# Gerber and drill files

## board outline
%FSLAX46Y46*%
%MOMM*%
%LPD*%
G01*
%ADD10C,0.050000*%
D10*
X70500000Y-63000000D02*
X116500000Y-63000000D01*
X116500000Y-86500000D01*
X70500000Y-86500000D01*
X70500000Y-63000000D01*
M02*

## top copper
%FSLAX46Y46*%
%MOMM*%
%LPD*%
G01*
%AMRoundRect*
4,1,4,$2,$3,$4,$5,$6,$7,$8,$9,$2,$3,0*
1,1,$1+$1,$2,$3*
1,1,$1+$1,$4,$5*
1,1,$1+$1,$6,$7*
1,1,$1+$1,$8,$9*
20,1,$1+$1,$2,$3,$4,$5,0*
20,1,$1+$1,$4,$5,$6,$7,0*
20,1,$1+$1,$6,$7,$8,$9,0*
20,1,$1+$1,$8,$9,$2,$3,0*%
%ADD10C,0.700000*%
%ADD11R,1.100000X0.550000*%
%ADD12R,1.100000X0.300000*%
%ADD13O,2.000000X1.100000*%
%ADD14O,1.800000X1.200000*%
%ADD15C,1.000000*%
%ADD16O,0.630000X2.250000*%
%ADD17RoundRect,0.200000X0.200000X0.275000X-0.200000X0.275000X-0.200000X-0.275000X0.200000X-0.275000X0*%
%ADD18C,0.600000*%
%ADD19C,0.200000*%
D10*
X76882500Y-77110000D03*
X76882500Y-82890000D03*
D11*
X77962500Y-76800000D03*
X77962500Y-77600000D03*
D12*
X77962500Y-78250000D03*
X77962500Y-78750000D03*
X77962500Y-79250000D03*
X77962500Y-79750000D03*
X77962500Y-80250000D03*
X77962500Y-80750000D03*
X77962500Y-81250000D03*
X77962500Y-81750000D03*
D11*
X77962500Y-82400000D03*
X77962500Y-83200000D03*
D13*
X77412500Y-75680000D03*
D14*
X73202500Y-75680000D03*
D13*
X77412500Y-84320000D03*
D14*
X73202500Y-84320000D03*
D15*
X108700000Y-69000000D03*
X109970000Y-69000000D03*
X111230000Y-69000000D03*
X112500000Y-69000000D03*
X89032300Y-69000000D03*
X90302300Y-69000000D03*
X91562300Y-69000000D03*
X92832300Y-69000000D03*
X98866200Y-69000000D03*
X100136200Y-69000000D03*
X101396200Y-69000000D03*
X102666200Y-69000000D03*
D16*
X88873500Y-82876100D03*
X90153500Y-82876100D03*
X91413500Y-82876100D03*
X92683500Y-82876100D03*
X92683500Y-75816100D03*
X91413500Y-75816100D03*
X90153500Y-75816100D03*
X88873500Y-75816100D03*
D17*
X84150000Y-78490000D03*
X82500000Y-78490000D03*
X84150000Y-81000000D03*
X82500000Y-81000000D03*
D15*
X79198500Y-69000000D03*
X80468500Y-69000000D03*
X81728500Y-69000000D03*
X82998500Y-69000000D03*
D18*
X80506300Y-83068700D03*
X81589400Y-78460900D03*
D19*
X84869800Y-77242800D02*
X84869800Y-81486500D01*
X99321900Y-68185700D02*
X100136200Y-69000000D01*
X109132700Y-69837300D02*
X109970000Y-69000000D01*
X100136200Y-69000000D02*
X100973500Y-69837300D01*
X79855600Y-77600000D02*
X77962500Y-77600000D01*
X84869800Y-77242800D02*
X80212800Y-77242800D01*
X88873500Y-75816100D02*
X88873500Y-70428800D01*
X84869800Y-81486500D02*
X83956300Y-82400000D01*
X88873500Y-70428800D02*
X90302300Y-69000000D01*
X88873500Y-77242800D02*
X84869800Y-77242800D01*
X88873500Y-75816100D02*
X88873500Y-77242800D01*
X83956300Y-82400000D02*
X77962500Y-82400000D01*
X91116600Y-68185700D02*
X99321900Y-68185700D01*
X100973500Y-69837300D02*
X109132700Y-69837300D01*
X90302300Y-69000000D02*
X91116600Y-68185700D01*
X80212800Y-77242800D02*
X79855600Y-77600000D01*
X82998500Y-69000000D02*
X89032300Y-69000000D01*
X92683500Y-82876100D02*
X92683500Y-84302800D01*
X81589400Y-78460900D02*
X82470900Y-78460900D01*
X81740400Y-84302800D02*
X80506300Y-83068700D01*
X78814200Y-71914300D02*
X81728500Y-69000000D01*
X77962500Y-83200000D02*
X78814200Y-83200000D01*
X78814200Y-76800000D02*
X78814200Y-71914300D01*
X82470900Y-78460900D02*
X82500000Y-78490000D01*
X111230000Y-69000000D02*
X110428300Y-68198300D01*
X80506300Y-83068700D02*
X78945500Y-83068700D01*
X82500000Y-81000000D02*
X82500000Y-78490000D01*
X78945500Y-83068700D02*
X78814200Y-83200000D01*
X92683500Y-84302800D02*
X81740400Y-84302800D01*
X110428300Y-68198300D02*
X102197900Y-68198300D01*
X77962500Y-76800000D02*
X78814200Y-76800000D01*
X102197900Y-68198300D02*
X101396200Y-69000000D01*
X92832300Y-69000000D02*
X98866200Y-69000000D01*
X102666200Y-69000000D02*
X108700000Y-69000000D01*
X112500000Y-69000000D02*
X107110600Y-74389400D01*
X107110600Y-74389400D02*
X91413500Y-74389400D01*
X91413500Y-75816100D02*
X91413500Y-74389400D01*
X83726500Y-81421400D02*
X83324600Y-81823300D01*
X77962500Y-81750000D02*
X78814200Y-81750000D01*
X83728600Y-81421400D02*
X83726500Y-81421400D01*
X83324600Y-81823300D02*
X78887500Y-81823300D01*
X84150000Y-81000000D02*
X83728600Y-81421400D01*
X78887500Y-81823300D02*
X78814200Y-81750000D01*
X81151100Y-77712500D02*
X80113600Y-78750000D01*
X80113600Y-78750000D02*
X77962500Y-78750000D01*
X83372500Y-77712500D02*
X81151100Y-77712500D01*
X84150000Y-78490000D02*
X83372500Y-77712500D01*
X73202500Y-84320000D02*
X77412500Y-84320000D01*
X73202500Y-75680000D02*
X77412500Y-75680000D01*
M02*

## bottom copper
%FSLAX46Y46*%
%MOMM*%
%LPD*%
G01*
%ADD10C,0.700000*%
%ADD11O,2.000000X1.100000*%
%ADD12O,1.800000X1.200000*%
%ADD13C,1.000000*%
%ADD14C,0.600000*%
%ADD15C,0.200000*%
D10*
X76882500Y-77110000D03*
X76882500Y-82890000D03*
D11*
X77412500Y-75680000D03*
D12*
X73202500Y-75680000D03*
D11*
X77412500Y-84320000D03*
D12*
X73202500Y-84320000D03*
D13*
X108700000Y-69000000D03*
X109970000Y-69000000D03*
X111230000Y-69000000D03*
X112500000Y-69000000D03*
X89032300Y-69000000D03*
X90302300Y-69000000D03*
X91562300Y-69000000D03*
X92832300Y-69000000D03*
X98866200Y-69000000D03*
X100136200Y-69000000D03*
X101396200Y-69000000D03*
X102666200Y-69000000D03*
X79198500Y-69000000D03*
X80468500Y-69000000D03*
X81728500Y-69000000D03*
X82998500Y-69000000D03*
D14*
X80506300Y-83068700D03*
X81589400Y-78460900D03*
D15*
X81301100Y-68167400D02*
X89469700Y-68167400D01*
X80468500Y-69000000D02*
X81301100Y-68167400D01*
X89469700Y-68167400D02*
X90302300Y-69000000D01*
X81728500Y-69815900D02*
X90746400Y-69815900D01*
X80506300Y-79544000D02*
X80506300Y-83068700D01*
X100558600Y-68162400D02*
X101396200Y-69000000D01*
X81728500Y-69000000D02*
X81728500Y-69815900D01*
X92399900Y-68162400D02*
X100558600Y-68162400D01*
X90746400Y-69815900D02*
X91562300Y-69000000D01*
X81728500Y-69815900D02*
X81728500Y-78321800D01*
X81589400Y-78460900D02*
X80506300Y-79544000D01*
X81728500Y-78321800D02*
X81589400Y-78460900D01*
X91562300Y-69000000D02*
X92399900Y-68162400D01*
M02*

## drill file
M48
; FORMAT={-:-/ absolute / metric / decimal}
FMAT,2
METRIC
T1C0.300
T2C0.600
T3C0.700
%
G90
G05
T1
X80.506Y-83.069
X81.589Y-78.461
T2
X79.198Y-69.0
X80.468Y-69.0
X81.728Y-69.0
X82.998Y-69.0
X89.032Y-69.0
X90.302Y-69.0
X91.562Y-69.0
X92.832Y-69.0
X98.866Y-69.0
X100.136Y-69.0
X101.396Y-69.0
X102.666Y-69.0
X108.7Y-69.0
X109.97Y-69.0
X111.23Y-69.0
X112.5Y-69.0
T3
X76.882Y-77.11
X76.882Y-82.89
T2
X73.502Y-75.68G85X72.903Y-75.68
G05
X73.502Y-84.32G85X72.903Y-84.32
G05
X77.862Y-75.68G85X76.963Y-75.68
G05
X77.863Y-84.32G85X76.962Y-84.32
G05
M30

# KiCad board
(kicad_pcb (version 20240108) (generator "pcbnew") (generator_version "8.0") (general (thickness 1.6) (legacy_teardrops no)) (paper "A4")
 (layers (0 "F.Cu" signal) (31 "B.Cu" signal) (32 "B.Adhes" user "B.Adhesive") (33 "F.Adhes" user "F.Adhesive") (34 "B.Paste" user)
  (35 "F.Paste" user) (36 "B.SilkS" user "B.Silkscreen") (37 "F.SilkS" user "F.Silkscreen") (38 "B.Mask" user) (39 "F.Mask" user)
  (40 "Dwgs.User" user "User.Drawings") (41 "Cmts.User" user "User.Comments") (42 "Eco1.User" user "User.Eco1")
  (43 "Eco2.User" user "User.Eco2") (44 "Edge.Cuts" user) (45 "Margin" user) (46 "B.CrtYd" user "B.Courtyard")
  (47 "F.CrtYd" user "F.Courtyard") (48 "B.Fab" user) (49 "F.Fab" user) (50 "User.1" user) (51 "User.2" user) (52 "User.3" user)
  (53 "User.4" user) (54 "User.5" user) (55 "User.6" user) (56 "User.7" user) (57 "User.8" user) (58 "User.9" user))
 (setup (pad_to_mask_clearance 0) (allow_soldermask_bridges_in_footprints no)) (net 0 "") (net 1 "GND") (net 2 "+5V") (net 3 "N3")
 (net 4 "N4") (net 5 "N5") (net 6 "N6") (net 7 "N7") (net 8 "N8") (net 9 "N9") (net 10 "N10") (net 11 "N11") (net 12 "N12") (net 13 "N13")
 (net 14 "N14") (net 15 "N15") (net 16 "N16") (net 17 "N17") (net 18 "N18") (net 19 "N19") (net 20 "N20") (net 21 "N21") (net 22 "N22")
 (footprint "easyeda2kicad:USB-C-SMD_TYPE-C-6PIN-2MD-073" (layer "F.Cu") (at 75.5825 80 -90)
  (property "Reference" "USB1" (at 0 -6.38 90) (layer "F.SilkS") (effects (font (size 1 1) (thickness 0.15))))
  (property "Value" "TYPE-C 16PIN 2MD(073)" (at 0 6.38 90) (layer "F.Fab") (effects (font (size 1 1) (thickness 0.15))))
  (pad "" thru_hole circle (at -2.89 -1.3 270) (size 0.7 0.7) (drill 0.7) (layers "*.Cu" "*.Mask") (remove_unused_layers no))
  (pad "" thru_hole circle (at 2.89 -1.3 270) (size 0.7 0.7) (drill 0.7) (layers "*.Cu" "*.Mask") (remove_unused_layers no))
  (pad "1" smd rect (at -3.2 -2.38 270) (size 0.55 1.1) (layers "F.Cu" "F.Paste" "F.Mask") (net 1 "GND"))
  (pad "2" smd rect (at -2.4 -2.38 270) (size 0.55 1.1) (layers "F.Cu" "F.Paste" "F.Mask") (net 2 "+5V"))
  (pad "3" smd rect (at -1.75 -2.38 270) (size 0.3 1.1) (layers "F.Cu" "F.Paste" "F.Mask") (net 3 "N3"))
  (pad "4" smd rect (at -1.25 -2.38 270) (size 0.3 1.1) (layers "F.Cu" "F.Paste" "F.Mask") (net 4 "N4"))
  (pad "5" smd rect (at -0.75 -2.38 270) (size 0.3 1.1) (layers "F.Cu" "F.Paste" "F.Mask") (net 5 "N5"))
  (pad "6" smd rect (at -0.25 -2.38 270) (size 0.3 1.1) (layers "F.Cu" "F.Paste" "F.Mask") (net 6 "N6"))
  (pad "7" smd rect (at 0.25 -2.38 270) (size 0.3 1.1) (layers "F.Cu" "F.Paste" "F.Mask") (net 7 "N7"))
  (pad "8" smd rect (at 0.75 -2.38 270) (size 0.3 1.1) (layers "F.Cu" "F.Paste" "F.Mask") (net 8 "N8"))
  (pad "9" smd rect (at 1.25 -2.38 270) (size 0.3 1.1) (layers "F.Cu" "F.Paste" "F.Mask") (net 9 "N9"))
  (pad "10" smd rect (at 1.75 -2.38 270) (size 0.3 1.1) (layers "F.Cu" "F.Paste" "F.Mask") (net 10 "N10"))
  (pad "11" smd rect (at 2.4 -2.38 270) (size 0.55 1.1) (layers "F.Cu" "F.Paste" "F.Mask") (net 2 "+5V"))
  (pad "12" smd rect (at 3.2 -2.38 270) (size 0.55 1.1) (layers "F.Cu" "F.Paste" "F.Mask") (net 1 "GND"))
  (pad "13" thru_hole oval (at -4.32 -1.83 270) (size 1.1 2) (drill oval 0.599999 1.499997) (layers "*.Cu" "*.Mask")
   (remove_unused_layers no) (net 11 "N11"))
  (pad "13" thru_hole oval (at -4.32 2.38 270) (size 1.2 1.8) (drill oval 0.599999 1.199998) (layers "*.Cu" "*.Mask")
   (remove_unused_layers no) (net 11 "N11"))
  (pad "14" thru_hole oval (at 4.32 -1.83 270) (size 1.1 2) (drill oval 0.599999 1.500022) (layers "*.Cu" "*.Mask")
   (remove_unused_layers no) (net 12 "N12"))
  (pad "14" thru_hole oval (at 4.32 2.38 270) (size 1.2 1.8) (drill oval 0.599999 1.199998) (layers "*.Cu" "*.Mask")
   (remove_unused_layers no) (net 12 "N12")))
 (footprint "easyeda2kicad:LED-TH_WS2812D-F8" (layer "F.Cu") (at 110.6 69)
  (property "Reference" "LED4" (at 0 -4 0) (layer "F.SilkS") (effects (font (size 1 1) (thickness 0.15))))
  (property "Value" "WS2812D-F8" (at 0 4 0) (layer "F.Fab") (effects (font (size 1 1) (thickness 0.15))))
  (pad "1" thru_hole circle (at -1.9 0) (size 1 1) (drill 0.599999) (layers "*.Cu" "*.Mask") (remove_unused_layers no) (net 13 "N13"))
  (pad "2" thru_hole circle (at -0.63 0) (size 1 1) (drill 0.599999) (layers "*.Cu" "*.Mask") (remove_unused_layers no) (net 2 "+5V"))
  (pad "3" thru_hole circle (at 0.63 0) (size 1 1) (drill 0.599999) (layers "*.Cu" "*.Mask") (remove_unused_layers no) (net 1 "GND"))
  (pad "4" thru_hole circle (at 1.9 0) (size 1 1) (drill 0.599999) (layers "*.Cu" "*.Mask") (remove_unused_layers no) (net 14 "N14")))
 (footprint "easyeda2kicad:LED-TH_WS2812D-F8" (layer "F.Cu") (at 90.9323 69)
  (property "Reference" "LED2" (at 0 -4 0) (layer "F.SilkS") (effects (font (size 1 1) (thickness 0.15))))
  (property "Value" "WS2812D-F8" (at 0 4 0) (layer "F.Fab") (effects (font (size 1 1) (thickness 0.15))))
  (pad "1" thru_hole circle (at -1.9 0) (size 1 1) (drill 0.599999) (layers "*.Cu" "*.Mask") (remove_unused_layers no) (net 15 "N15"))
  (pad "2" thru_hole circle (at -0.63 0) (size 1 1) (drill 0.599999) (layers "*.Cu" "*.Mask") (remove_unused_layers no) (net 2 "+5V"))
  (pad "3" thru_hole circle (at 0.63 0) (size 1 1) (drill 0.599999) (layers "*.Cu" "*.Mask") (remove_unused_layers no) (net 1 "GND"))
  (pad "4" thru_hole circle (at 1.9 0) (size 1 1) (drill 0.599999) (layers "*.Cu" "*.Mask") (remove_unused_layers no) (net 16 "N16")))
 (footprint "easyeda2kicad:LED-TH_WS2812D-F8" (layer "F.Cu") (at 100.7662 69)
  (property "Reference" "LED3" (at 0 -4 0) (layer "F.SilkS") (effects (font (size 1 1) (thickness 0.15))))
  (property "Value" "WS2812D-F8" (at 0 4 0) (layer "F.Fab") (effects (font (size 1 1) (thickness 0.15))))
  (pad "1" thru_hole circle (at -1.9 0) (size 1 1) (drill 0.599999) (layers "*.Cu" "*.Mask") (remove_unused_layers no) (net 16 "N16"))
  (pad "2" thru_hole circle (at -0.63 0) (size 1 1) (drill 0.599999) (layers "*.Cu" "*.Mask") (remove_unused_layers no) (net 2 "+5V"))
  (pad "3" thru_hole circle (at 0.63 0) (size 1 1) (drill 0.599999) (layers "*.Cu" "*.Mask") (remove_unused_layers no) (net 1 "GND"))
  (pad "4" thru_hole circle (at 1.9 0) (size 1 1) (drill 0.599999) (layers "*.Cu" "*.Mask") (remove_unused_layers no) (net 13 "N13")))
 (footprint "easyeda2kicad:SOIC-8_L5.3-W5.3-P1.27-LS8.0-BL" (layer "F.Cu") (at 90.7835 79.3461)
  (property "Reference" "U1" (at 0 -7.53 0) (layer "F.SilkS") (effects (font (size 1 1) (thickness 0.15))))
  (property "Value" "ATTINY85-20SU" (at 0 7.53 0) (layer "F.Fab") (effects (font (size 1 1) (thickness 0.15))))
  (pad "1" smd oval (at -1.91 3.53) (size 0.63 2.25) (layers "F.Cu" "F.Paste" "F.Mask") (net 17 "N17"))
  (pad "2" smd oval (at -0.63 3.53) (size 0.63 2.25) (layers "F.Cu" "F.Paste" "F.Mask") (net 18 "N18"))
  (pad "3" smd oval (at 0.63 3.53) (size 0.63 2.25) (layers "F.Cu" "F.Paste" "F.Mask") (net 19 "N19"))
  (pad "4" smd oval (at 1.9 3.53) (size 0.63 2.25) (layers "F.Cu" "F.Paste" "F.Mask") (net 1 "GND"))
  (pad "5" smd oval (at 1.9 -3.53) (size 0.63 2.25) (layers "F.Cu" "F.Paste" "F.Mask") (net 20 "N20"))
  (pad "6" smd oval (at 0.63 -3.53) (size 0.63 2.25) (layers "F.Cu" "F.Paste" "F.Mask") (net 14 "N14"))
  (pad "7" smd oval (at -0.63 -3.53) (size 0.63 2.25) (layers "F.Cu" "F.Paste" "F.Mask") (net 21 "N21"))
  (pad "8" smd oval (at -1.91 -3.53) (size 0.63 2.25) (layers "F.Cu" "F.Paste" "F.Mask") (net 2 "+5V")))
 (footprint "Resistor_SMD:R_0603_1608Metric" (layer "F.Cu") (at 83.325 78.49 180)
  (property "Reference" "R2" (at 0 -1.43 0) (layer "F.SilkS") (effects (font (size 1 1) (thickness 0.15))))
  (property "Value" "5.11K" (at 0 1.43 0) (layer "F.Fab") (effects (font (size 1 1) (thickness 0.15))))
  (pad "1" smd roundrect (at -0.825 0 180) (size 0.8 0.95) (layers "F.Cu" "F.Paste" "F.Mask") (roundrect_rratio 0.25) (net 4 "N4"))
  (pad "2" smd roundrect (at 0.825 0 180) (size 0.8 0.95) (layers "F.Cu" "F.Paste" "F.Mask") (roundrect_rratio 0.25) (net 1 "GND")))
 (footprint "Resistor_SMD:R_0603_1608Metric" (layer "F.Cu") (at 83.325 81 180)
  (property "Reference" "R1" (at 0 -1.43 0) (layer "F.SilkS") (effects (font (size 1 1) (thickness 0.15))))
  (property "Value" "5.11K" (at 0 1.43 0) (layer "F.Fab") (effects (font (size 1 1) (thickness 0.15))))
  (pad "1" smd roundrect (at -0.825 0 180) (size 0.8 0.95) (layers "F.Cu" "F.Paste" "F.Mask") (roundrect_rratio 0.25) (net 10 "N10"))
  (pad "2" smd roundrect (at 0.825 0 180) (size 0.8 0.95) (layers "F.Cu" "F.Paste" "F.Mask") (roundrect_rratio 0.25) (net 1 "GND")))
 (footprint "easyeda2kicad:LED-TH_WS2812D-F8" (layer "F.Cu") (at 81.0985 69)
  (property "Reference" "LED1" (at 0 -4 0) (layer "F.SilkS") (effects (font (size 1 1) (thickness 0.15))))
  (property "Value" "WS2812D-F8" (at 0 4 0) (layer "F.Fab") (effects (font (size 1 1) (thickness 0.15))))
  (pad "1" thru_hole circle (at -1.9 0) (size 1 1) (drill 0.599999) (layers "*.Cu" "*.Mask") (remove_unused_layers no) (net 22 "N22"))
  (pad "2" thru_hole circle (at -0.63 0) (size 1 1) (drill 0.599999) (layers "*.Cu" "*.Mask") (remove_unused_layers no) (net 2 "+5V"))
  (pad "3" thru_hole circle (at 0.63 0) (size 1 1) (drill 0.599999) (layers "*.Cu" "*.Mask") (remove_unused_layers no) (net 1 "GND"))
  (pad "4" thru_hole circle (at 1.9 0) (size 1 1) (drill 0.599999) (layers "*.Cu" "*.Mask") (remove_unused_layers no) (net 15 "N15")))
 (gr_rect (start 70.5 63) (end 116.5 86.5) (stroke (width 0.05) (type default)) (fill none) (layer "Edge.Cuts"))
 (segment (start 84.8698 77.2428) (end 84.8698 81.4865) (width 0.2) (layer "F.Cu") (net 2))
 (segment (start 99.3219 68.1857) (end 100.1362 69) (width 0.2) (layer "F.Cu") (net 2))
 (segment (start 109.1327 69.8373) (end 109.97 69) (width 0.2) (layer "F.Cu") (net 2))
 (segment (start 100.1362 69) (end 100.9735 69.8373) (width 0.2) (layer "F.Cu") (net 2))
 (segment (start 79.8556 77.6) (end 77.9625 77.6) (width 0.2) (layer "F.Cu") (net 2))
 (segment (start 84.8698 77.2428) (end 80.2128 77.2428) (width 0.2) (layer "F.Cu") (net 2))
 (segment (start 88.8735 75.8161) (end 88.8735 70.4288) (width 0.2) (layer "F.Cu") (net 2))
 (segment (start 84.8698 81.4865) (end 83.9563 82.4) (width 0.2) (layer "F.Cu") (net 2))
 (segment (start 88.8735 70.4288) (end 90.3023 69) (width 0.2) (layer "F.Cu") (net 2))
 (segment (start 88.8735 77.2428) (end 84.8698 77.2428) (width 0.2) (layer "F.Cu") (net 2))
 (segment (start 88.8735 75.8161) (end 88.8735 77.2428) (width 0.2) (layer "F.Cu") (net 2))
 (segment (start 83.9563 82.4) (end 77.9625 82.4) (width 0.2) (layer "F.Cu") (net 2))
 (segment (start 91.1166 68.1857) (end 99.3219 68.1857) (width 0.2) (layer "F.Cu") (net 2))
 (segment (start 100.9735 69.8373) (end 109.1327 69.8373) (width 0.2) (layer "F.Cu") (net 2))
 (segment (start 90.3023 69) (end 91.1166 68.1857) (width 0.2) (layer "F.Cu") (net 2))
 (segment (start 80.2128 77.2428) (end 79.8556 77.6) (width 0.2) (layer "F.Cu") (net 2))
 (segment (start 81.3011 68.1674) (end 89.4697 68.1674) (width 0.2) (layer "B.Cu") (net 2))
 (segment (start 80.4685 69) (end 81.3011 68.1674) (width 0.2) (layer "B.Cu") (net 2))
 (segment (start 89.4697 68.1674) (end 90.3023 69) (width 0.2) (layer "B.Cu") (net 2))
 (segment (start 82.9985 69) (end 89.0323 69) (width 0.2) (layer "F.Cu") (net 15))
 (segment (start 92.6835 82.8761) (end 92.6835 84.3028) (width 0.2) (layer "F.Cu") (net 1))
 (segment (start 81.5894 78.4609) (end 82.4709 78.4609) (width 0.2) (layer "F.Cu") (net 1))
 (segment (start 81.7404 84.3028) (end 80.5063 83.0687) (width 0.2) (layer "F.Cu") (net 1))
 (segment (start 78.8142 71.9143) (end 81.7285 69) (width 0.2) (layer "F.Cu") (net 1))
 (segment (start 77.9625 83.2) (end 78.8142 83.2) (width 0.2) (layer "F.Cu") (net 1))
 (segment (start 78.8142 76.8) (end 78.8142 71.9143) (width 0.2) (layer "F.Cu") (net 1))
 (segment (start 82.4709 78.4609) (end 82.5 78.49) (width 0.2) (layer "F.Cu") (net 1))
 (segment (start 111.23 69) (end 110.4283 68.1983) (width 0.2) (layer "F.Cu") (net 1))
 (segment (start 80.5063 83.0687) (end 78.9455 83.0687) (width 0.2) (layer "F.Cu") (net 1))
 (segment (start 82.5 81) (end 82.5 78.49) (width 0.2) (layer "F.Cu") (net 1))
 (segment (start 78.9455 83.0687) (end 78.8142 83.2) (width 0.2) (layer "F.Cu") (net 1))
 (segment (start 92.6835 84.3028) (end 81.7404 84.3028) (width 0.2) (layer "F.Cu") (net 1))
 (segment (start 110.4283 68.1983) (end 102.1979 68.1983) (width 0.2) (layer "F.Cu") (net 1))
 (segment (start 77.9625 76.8) (end 78.8142 76.8) (width 0.2) (layer "F.Cu") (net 1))
 (segment (start 102.1979 68.1983) (end 101.3962 69) (width 0.2) (layer "F.Cu") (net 1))
 (via (at 80.5063 83.0687) (size 0.6) (drill 0.3) (layers "F.Cu" "B.Cu") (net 1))
 (via (at 81.5894 78.4609) (size 0.6) (drill 0.3) (layers "F.Cu" "B.Cu") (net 1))
 (segment (start 81.7285 69.8159) (end 90.7464 69.8159) (width 0.2) (layer "B.Cu") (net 1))
 (segment (start 80.5063 79.544) (end 80.5063 83.0687) (width 0.2) (layer "B.Cu") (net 1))
 (segment (start 100.5586 68.1624) (end 101.3962 69) (width 0.2) (layer "B.Cu") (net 1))
 (segment (start 81.7285 69) (end 81.7285 69.8159) (width 0.2) (layer "B.Cu") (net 1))
 (segment (start 92.3999 68.1624) (end 100.5586 68.1624) (width 0.2) (layer "B.Cu") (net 1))
 (segment (start 90.7464 69.8159) (end 91.5623 69) (width 0.2) (layer "B.Cu") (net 1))
 (segment (start 81.7285 69.8159) (end 81.7285 78.3218) (width 0.2) (layer "B.Cu") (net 1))
 (segment (start 81.5894 78.4609) (end 80.5063 79.544) (width 0.2) (layer "B.Cu") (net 1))
 (segment (start 81.7285 78.3218) (end 81.5894 78.4609) (width 0.2) (layer "B.Cu") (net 1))
 (segment (start 91.5623 69) (end 92.3999 68.1624) (width 0.2) (layer "B.Cu") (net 1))
 (segment (start 92.8323 69) (end 98.8662 69) (width 0.2) (layer "F.Cu") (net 16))
 (segment (start 102.6662 69) (end 108.7 69) (width 0.2) (layer "F.Cu") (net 13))
 (segment (start 112.5 69) (end 107.1106 74.3894) (width 0.2) (layer "F.Cu") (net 14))
 (segment (start 107.1106 74.3894) (end 91.4135 74.3894) (width 0.2) (layer "F.Cu") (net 14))
 (segment (start 91.4135 75.8161) (end 91.4135 74.3894) (width 0.2) (layer "F.Cu") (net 14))
 (segment (start 83.7265 81.4214) (end 83.3246 81.8233) (width 0.2) (layer "F.Cu") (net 10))
 (segment (start 77.9625 81.75) (end 78.8142 81.75) (width 0.2) (layer "F.Cu") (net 10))
 (segment (start 83.7286 81.4214) (end 83.7265 81.4214) (width 0.2) (layer "F.Cu") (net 10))
 (segment (start 83.3246 81.8233) (end 78.8875 81.8233) (width 0.2) (layer "F.Cu") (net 10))
 (segment (start 84.15 81) (end 83.7286 81.4214) (width 0.2) (layer "F.Cu") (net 10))
 (segment (start 78.8875 81.8233) (end 78.8142 81.75) (width 0.2) (layer "F.Cu") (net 10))
 (segment (start 81.1511 77.7125) (end 80.1136 78.75) (width 0.2) (layer "F.Cu") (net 4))
 (segment (start 80.1136 78.75) (end 77.9625 78.75) (width 0.2) (layer "F.Cu") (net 4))
 (segment (start 83.3725 77.7125) (end 81.1511 77.7125) (width 0.2) (layer "F.Cu") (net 4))
 (segment (start 84.15 78.49) (end 83.3725 77.7125) (width 0.2) (layer "F.Cu") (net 4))
 (segment (start 73.2025 84.32) (end 77.4125 84.32) (width 0.2) (layer "F.Cu") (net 12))
 (segment (start 73.2025 75.68) (end 77.4125 75.68) (width 0.2) (layer "F.Cu") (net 11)))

